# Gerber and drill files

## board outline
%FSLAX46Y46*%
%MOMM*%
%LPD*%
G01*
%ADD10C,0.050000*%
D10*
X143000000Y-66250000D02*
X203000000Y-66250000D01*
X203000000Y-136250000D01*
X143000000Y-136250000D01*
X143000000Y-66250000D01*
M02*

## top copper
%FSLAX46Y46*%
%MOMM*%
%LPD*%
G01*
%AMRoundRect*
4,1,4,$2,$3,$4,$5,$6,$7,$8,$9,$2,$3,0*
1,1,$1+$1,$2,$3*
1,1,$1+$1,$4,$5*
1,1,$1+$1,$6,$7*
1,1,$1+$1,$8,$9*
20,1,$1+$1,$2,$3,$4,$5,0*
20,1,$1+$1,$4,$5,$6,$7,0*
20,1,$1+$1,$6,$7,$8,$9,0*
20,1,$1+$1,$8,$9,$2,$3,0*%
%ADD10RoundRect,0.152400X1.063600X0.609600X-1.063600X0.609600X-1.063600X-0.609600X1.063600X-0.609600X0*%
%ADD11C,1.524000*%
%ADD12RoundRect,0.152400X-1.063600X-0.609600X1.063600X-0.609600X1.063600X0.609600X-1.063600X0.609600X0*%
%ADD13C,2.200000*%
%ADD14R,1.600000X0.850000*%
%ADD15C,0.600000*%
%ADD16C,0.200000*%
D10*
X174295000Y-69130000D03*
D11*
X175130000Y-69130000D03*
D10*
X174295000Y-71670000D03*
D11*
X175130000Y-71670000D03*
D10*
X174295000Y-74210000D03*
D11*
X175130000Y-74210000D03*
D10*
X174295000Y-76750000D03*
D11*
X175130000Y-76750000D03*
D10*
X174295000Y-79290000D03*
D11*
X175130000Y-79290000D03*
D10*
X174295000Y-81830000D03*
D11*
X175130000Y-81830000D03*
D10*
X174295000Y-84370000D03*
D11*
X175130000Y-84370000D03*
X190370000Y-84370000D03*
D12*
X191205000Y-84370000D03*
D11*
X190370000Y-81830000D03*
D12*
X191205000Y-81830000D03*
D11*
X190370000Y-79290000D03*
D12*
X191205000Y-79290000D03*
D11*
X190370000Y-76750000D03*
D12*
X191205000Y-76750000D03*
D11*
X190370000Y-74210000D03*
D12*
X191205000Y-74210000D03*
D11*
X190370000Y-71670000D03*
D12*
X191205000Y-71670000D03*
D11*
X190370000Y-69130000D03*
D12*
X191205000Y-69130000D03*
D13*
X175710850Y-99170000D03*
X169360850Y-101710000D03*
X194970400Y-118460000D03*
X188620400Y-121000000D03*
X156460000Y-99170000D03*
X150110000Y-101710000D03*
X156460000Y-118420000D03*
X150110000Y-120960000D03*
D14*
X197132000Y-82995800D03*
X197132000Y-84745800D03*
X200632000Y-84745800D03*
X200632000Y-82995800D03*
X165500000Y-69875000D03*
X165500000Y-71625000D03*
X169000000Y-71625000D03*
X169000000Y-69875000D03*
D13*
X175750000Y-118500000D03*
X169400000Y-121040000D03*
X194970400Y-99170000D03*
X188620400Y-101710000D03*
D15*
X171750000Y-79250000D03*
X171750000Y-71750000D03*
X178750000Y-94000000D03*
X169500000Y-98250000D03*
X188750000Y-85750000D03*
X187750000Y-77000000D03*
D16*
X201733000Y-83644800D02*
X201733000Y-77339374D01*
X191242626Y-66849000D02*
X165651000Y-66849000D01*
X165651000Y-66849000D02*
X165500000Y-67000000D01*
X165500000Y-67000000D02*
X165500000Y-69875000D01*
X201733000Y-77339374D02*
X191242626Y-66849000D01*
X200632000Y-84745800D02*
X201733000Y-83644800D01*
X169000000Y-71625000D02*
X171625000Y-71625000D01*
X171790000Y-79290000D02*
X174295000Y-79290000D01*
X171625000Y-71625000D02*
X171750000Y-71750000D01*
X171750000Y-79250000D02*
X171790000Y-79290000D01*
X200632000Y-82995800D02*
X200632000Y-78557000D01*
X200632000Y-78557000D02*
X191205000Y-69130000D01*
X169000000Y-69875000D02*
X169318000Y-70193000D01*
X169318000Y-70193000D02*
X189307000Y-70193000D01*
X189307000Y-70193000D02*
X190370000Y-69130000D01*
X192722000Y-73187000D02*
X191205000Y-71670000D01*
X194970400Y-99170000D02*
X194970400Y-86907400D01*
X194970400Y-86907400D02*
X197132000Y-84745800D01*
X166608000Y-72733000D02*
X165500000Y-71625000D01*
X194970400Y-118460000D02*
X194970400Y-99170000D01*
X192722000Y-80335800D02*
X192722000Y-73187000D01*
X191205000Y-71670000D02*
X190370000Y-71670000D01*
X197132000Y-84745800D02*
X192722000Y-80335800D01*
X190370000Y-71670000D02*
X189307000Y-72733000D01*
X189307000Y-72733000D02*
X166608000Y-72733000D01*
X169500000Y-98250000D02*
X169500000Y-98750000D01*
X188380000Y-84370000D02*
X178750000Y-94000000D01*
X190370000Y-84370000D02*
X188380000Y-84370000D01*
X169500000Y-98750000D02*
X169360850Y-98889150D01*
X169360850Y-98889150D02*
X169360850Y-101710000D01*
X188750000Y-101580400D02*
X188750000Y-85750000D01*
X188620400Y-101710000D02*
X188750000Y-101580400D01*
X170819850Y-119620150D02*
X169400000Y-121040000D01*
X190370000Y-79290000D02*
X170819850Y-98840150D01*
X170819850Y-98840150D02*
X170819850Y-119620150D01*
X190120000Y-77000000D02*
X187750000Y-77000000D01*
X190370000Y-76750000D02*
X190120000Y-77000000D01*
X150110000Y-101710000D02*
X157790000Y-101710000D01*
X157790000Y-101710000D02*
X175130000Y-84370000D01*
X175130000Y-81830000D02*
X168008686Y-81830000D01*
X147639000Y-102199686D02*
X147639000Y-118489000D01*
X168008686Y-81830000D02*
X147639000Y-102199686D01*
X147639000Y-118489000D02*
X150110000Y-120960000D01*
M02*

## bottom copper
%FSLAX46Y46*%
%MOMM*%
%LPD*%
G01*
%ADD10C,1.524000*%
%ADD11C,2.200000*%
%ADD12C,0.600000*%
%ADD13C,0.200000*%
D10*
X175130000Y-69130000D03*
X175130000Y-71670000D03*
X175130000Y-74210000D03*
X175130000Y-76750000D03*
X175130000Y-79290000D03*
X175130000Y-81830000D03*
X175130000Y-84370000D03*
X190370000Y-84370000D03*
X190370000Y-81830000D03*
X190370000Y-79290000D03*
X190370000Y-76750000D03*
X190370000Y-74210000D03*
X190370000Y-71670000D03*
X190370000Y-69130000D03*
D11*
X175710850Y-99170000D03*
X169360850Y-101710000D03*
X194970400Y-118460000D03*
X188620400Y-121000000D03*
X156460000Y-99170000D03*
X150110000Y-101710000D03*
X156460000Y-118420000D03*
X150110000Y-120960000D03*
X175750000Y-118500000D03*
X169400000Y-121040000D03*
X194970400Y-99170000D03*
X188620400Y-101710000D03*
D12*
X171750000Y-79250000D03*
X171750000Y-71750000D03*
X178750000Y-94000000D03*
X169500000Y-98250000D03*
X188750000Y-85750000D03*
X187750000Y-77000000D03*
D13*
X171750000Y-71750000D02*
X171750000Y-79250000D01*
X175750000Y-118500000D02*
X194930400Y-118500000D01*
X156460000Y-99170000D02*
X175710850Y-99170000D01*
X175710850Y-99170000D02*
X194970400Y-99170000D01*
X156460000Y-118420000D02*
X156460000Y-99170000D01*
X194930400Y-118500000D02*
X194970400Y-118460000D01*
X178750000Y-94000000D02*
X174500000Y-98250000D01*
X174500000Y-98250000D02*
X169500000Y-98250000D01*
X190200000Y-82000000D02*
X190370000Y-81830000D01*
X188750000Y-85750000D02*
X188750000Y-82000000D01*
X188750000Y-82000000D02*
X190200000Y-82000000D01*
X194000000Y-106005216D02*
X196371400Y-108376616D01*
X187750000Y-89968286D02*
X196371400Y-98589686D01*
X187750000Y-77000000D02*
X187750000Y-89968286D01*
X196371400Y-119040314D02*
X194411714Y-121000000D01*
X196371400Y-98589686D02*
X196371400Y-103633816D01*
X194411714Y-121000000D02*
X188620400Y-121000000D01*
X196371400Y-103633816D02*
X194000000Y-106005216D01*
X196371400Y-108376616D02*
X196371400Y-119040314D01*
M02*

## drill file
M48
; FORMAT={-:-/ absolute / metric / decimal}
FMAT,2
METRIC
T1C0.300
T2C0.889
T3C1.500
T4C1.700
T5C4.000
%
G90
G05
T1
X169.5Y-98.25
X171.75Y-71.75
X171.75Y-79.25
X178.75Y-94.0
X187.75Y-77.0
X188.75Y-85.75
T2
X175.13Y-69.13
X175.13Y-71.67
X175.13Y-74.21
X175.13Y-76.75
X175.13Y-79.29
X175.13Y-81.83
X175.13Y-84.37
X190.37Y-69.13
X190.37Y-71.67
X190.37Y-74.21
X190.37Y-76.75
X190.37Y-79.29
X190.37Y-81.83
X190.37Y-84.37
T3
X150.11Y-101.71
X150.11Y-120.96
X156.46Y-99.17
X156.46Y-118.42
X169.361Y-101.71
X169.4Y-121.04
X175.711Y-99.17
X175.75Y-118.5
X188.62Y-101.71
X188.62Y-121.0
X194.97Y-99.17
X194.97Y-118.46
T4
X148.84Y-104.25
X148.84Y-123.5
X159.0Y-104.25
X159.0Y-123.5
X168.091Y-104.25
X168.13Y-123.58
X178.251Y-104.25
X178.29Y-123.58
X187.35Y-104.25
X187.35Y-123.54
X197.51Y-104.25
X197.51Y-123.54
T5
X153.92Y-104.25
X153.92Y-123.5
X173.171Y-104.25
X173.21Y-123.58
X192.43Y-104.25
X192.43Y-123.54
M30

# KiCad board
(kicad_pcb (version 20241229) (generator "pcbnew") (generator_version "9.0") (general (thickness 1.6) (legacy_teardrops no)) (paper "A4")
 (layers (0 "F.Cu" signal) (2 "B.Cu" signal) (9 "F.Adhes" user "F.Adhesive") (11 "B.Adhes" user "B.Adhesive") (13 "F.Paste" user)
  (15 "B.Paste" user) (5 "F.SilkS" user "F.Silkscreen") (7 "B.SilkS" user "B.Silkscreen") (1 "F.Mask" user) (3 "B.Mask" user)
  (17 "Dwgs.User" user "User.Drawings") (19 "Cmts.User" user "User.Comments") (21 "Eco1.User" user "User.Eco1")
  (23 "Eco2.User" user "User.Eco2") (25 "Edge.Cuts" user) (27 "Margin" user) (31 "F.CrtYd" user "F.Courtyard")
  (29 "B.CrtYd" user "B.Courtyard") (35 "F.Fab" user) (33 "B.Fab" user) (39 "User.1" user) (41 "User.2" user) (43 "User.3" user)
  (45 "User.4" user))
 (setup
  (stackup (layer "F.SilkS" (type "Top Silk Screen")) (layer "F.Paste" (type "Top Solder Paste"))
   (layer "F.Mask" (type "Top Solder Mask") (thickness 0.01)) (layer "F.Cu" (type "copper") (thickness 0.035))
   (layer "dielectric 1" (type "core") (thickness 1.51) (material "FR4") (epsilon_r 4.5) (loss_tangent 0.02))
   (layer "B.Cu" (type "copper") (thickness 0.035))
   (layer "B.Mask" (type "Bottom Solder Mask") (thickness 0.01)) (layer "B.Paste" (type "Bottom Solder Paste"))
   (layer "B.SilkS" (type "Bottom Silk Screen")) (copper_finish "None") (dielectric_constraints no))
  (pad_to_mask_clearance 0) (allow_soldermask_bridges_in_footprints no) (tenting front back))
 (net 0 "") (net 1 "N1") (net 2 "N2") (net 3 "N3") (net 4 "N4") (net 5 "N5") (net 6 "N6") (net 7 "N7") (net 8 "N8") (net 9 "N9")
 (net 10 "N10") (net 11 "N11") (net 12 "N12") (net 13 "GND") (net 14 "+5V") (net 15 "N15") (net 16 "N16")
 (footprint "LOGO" (layer "F.Cu") (at 198.75 69.5)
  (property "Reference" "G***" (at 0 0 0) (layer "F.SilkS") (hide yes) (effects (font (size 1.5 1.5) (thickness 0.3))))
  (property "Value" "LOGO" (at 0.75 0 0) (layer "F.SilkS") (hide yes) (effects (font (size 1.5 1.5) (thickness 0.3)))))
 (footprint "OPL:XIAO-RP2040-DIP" (layer "F.Cu") (at 182.75 76.75)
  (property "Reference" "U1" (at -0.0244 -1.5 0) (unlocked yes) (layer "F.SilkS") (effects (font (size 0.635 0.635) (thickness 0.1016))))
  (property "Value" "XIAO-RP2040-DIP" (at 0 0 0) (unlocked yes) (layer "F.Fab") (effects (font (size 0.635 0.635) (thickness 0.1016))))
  (pad "1" smd roundrect (at -8.455 -7.62 180) (size 2.432 1.524) (layers "F.Cu" "F.Mask") (roundrect_rratio 0.1) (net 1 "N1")
   (thermal_bridge_angle 45))
  (pad "1" thru_hole circle (at -7.62 -7.62 180) (size 1.524 1.524) (drill 0.889) (layers "*.Cu" "*.Mask") (remove_unused_layers no)
   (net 1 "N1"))
  (pad "2" smd roundrect (at -8.455 -5.08 180) (size 2.432 1.524) (layers "F.Cu" "F.Mask") (roundrect_rratio 0.1) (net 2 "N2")
   (thermal_bridge_angle 45))
  (pad "2" thru_hole circle (at -7.62 -5.08 180) (size 1.524 1.524) (drill 0.889) (layers "*.Cu" "*.Mask") (remove_unused_layers no)
   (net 2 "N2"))
  (pad "3" smd roundrect (at -8.455 -2.54 180) (size 2.432 1.524) (layers "F.Cu" "F.Mask") (roundrect_rratio 0.1) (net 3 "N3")
   (thermal_bridge_angle 45))
  (pad "3" thru_hole circle (at -7.62 -2.54 180) (size 1.524 1.524) (drill 0.889) (layers "*.Cu" "*.Mask") (remove_unused_layers no)
   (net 3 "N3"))
  (pad "4" smd roundrect (at -8.455 0 180) (size 2.432 1.524) (layers "F.Cu" "F.Mask") (roundrect_rratio 0.1) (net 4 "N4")
   (thermal_bridge_angle 45))
  (pad "4" thru_hole circle (at -7.62 0 180) (size 1.524 1.524) (drill 0.889) (layers "*.Cu" "*.Mask") (remove_unused_layers no)
   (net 4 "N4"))
  (pad "5" smd roundrect (at -8.455 2.54 180) (size 2.432 1.524) (layers "F.Cu" "F.Mask") (roundrect_rratio 0.1) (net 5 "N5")
   (thermal_bridge_angle 45))
  (pad "5" thru_hole circle (at -7.62 2.54 180) (size 1.524 1.524) (drill 0.889) (layers "*.Cu" "*.Mask") (remove_unused_layers no)
   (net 5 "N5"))
  (pad "6" smd roundrect (at -8.455 5.08 180) (size 2.432 1.524) (layers "F.Cu" "F.Mask") (roundrect_rratio 0.1) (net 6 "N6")
   (thermal_bridge_angle 45))
  (pad "6" thru_hole circle (at -7.62 5.08 180) (size 1.524 1.524) (drill 0.889) (layers "*.Cu" "*.Mask") (remove_unused_layers no)
   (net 6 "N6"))
  (pad "7" smd roundrect (at -8.455 7.62 180) (size 2.432 1.524) (layers "F.Cu" "F.Mask") (roundrect_rratio 0.1) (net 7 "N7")
   (thermal_bridge_angle 45))
  (pad "7" thru_hole circle (at -7.62 7.62 180) (size 1.524 1.524) (drill 0.889) (layers "*.Cu" "*.Mask") (remove_unused_layers no)
   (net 7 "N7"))
  (pad "8" thru_hole circle (at 7.62 7.62) (size 1.524 1.524) (drill 0.889) (layers "*.Cu" "*.Mask") (remove_unused_layers no) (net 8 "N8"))
  (pad "8" smd roundrect (at 8.455 7.62) (size 2.432 1.524) (layers "F.Cu" "F.Mask") (roundrect_rratio 0.1) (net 8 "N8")
   (thermal_bridge_angle 45))
  (pad "9" thru_hole circle (at 7.62 5.08) (size 1.524 1.524) (drill 0.889) (layers "*.Cu" "*.Mask") (remove_unused_layers no) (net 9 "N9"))
  (pad "9" smd roundrect (at 8.455 5.08) (size 2.432 1.524) (layers "F.Cu" "F.Mask") (roundrect_rratio 0.1) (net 9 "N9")
   (thermal_bridge_angle 45))
  (pad "10" thru_hole circle (at 7.62 2.54) (size 1.524 1.524) (drill 0.889) (layers "*.Cu" "*.Mask") (remove_unused_layers no)
   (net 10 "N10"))
  (pad "10" smd roundrect (at 8.455 2.54) (size 2.432 1.524) (layers "F.Cu" "F.Mask") (roundrect_rratio 0.1) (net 10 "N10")
   (thermal_bridge_angle 45))
  (pad "11" thru_hole circle (at 7.62 0) (size 1.524 1.524) (drill 0.889) (layers "*.Cu" "*.Mask") (remove_unused_layers no) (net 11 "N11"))
  (pad "11" smd roundrect (at 8.455 0) (size 2.432 1.524) (layers "F.Cu" "F.Mask") (roundrect_rratio 0.1) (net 11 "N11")
   (thermal_bridge_angle 45))
  (pad "12" thru_hole circle (at 7.62 -2.54) (size 1.524 1.524) (drill 0.889) (layers "*.Cu" "*.Mask") (remove_unused_layers no)
   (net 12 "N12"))
  (pad "12" smd roundrect (at 8.455 -2.54) (size 2.432 1.524) (layers "F.Cu" "F.Mask") (roundrect_rratio 0.1) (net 12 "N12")
   (thermal_bridge_angle 45))
  (pad "13" thru_hole circle (at 7.62 -5.08) (size 1.524 1.524) (drill 0.889) (layers "*.Cu" "*.Mask") (remove_unused_layers no)
   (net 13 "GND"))
  (pad "13" smd roundrect (at 8.455 -5.08) (size 2.432 1.524) (layers "F.Cu" "F.Mask") (roundrect_rratio 0.1) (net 13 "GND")
   (thermal_bridge_angle 45))
  (pad "14" thru_hole circle (at 7.62 -7.62) (size 1.524 1.524) (drill 0.889) (layers "*.Cu" "*.Mask") (remove_unused_layers no)
   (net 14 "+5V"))
  (pad "14" smd roundrect (at 8.455 -7.62) (size 2.432 1.524) (layers "F.Cu" "F.Mask") (roundrect_rratio 0.1) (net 14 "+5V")
   (thermal_bridge_angle 45)))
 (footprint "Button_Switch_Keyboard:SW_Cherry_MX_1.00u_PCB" (layer "F.Cu") (at 175.71085 99.17)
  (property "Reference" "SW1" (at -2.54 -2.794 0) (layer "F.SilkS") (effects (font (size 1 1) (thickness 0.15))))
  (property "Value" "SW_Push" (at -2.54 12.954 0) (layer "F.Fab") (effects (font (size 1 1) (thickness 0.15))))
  (pad "" np_thru_hole circle (at -7.62 5.08) (size 1.7 1.7) (drill 1.7) (layers "*.Cu" "*.Mask"))
  (pad "" np_thru_hole circle (at -2.54 5.08) (size 4 4) (drill 4) (layers "*.Cu" "*.Mask"))
  (pad "" np_thru_hole circle (at 2.54 5.08) (size 1.7 1.7) (drill 1.7) (layers "*.Cu" "*.Mask"))
  (pad "1" thru_hole circle (at 0 0) (size 2.2 2.2) (drill 1.5) (layers "*.Cu" "*.Mask") (remove_unused_layers no) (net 13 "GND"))
  (pad "2" thru_hole circle (at -6.35 2.54) (size 2.2 2.2) (drill 1.5) (layers "*.Cu" "*.Mask") (remove_unused_layers no) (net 8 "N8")))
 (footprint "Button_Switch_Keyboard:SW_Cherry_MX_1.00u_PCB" (layer "F.Cu") (at 194.9704 118.46)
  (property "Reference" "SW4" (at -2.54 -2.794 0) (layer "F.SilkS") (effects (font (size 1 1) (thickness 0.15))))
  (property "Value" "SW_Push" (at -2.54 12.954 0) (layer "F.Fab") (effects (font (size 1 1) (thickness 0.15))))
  (pad "" np_thru_hole circle (at -7.62 5.08) (size 1.7 1.7) (drill 1.7) (layers "*.Cu" "*.Mask"))
  (pad "" np_thru_hole circle (at -2.54 5.08) (size 4 4) (drill 4) (layers "*.Cu" "*.Mask"))
  (pad "" np_thru_hole circle (at 2.54 5.08) (size 1.7 1.7) (drill 1.7) (layers "*.Cu" "*.Mask"))
  (pad "1" thru_hole circle (at 0 0) (size 2.2 2.2) (drill 1.5) (layers "*.Cu" "*.Mask") (remove_unused_layers no) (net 13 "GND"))
  (pad "2" thru_hole circle (at -6.35 2.54) (size 2.2 2.2) (drill 1.5) (layers "*.Cu" "*.Mask") (remove_unused_layers no) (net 11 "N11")))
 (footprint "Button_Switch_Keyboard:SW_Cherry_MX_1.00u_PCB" (layer "F.Cu") (at 156.46 99.17)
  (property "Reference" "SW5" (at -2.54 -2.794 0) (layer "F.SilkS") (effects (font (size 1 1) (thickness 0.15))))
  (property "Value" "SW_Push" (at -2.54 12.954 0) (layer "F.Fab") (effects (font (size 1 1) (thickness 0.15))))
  (pad "" np_thru_hole circle (at -7.62 5.08) (size 1.7 1.7) (drill 1.7) (layers "*.Cu" "*.Mask"))
  (pad "" np_thru_hole circle (at -2.54 5.08) (size 4 4) (drill 4) (layers "*.Cu" "*.Mask"))
  (pad "" np_thru_hole circle (at 2.54 5.08) (size 1.7 1.7) (drill 1.7) (layers "*.Cu" "*.Mask"))
  (pad "1" thru_hole circle (at 0 0) (size 2.2 2.2) (drill 1.5) (layers "*.Cu" "*.Mask") (remove_unused_layers no) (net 13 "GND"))
  (pad "2" thru_hole circle (at -6.35 2.54) (size 2.2 2.2) (drill 1.5) (layers "*.Cu" "*.Mask") (remove_unused_layers no) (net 7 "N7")))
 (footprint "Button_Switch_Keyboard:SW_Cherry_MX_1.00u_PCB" (layer "F.Cu") (at 156.46 118.42)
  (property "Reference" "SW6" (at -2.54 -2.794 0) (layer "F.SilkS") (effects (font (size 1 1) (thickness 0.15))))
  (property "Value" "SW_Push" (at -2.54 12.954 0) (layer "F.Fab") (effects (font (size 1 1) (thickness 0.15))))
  (pad "" np_thru_hole circle (at -7.62 5.08) (size 1.7 1.7) (drill 1.7) (layers "*.Cu" "*.Mask"))
  (pad "" np_thru_hole circle (at -2.54 5.08) (size 4 4) (drill 4) (layers "*.Cu" "*.Mask"))
  (pad "" np_thru_hole circle (at 2.54 5.08) (size 1.7 1.7) (drill 1.7) (layers "*.Cu" "*.Mask"))
  (pad "1" thru_hole circle (at 0 0) (size 2.2 2.2) (drill 1.5) (layers "*.Cu" "*.Mask") (remove_unused_layers no) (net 13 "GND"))
  (pad "2" thru_hole circle (at -6.35 2.54) (size 2.2 2.2) (drill 1.5) (layers "*.Cu" "*.Mask") (remove_unused_layers no) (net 6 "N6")))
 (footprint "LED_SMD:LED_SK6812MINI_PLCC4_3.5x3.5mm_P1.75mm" (layer "F.Cu") (at 198.882 83.8708)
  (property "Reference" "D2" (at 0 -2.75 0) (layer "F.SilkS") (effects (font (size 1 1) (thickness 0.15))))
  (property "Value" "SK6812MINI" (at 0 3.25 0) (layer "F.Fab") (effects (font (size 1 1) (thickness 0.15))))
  (pad "1" smd rect (at -1.75 -0.875) (size 1.6 0.85) (layers "F.Cu" "F.Mask" "F.Paste") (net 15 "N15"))
  (pad "2" smd rect (at -1.75 0.875) (size 1.6 0.85) (layers "F.Cu" "F.Mask" "F.Paste") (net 13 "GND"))
  (pad "3" smd rect (at 1.75 0.875) (size 1.6 0.85) (layers "F.Cu" "F.Mask" "F.Paste") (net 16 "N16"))
  (pad "4" smd rect (at 1.75 -0.875) (size 1.6 0.85) (layers "F.Cu" "F.Mask" "F.Paste") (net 14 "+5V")))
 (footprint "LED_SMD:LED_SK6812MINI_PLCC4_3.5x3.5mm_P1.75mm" (layer "F.Cu") (at 167.25 70.75)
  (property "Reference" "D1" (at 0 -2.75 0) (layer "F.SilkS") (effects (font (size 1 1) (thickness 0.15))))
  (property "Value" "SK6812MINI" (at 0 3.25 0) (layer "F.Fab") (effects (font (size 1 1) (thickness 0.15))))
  (pad "1" smd rect (at -1.75 -0.875) (size 1.6 0.85) (layers "F.Cu" "F.Mask" "F.Paste") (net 16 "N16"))
  (pad "2" smd rect (at -1.75 0.875) (size 1.6 0.85) (layers "F.Cu" "F.Mask" "F.Paste") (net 13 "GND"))
  (pad "3" smd rect (at 1.75 0.875) (size 1.6 0.85) (layers "F.Cu" "F.Mask" "F.Paste") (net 5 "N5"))
  (pad "4" smd rect (at 1.75 -0.875) (size 1.6 0.85) (layers "F.Cu" "F.Mask" "F.Paste") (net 14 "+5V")))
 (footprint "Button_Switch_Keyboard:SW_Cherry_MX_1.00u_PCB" (layer "F.Cu") (at 175.75 118.5)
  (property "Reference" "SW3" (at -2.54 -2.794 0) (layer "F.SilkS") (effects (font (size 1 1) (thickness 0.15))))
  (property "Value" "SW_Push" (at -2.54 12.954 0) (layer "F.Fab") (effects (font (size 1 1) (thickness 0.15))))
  (pad "" np_thru_hole circle (at -7.62 5.08) (size 1.7 1.7) (drill 1.7) (layers "*.Cu" "*.Mask"))
  (pad "" np_thru_hole circle (at -2.54 5.08) (size 4 4) (drill 4) (layers "*.Cu" "*.Mask"))
  (pad "" np_thru_hole circle (at 2.54 5.08) (size 1.7 1.7) (drill 1.7) (layers "*.Cu" "*.Mask"))
  (pad "1" thru_hole circle (at 0 0) (size 2.2 2.2) (drill 1.5) (layers "*.Cu" "*.Mask") (remove_unused_layers no) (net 13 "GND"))
  (pad "2" thru_hole circle (at -6.35 2.54) (size 2.2 2.2) (drill 1.5) (layers "*.Cu" "*.Mask") (remove_unused_layers no) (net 10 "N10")))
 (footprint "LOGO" (layer "F.Cu") (at 147.25 72)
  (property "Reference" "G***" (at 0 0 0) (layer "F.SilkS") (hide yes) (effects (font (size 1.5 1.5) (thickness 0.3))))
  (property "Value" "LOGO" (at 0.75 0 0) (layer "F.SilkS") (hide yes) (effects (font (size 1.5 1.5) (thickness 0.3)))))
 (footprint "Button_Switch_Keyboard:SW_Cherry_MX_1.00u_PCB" (layer "F.Cu") (at 194.9704 99.17)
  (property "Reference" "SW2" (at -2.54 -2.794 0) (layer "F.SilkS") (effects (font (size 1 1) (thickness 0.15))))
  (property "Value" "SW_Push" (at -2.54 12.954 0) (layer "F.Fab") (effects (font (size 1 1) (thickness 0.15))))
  (pad "" np_thru_hole circle (at -7.62 5.08) (size 1.7 1.7) (drill 1.7) (layers "*.Cu" "*.Mask"))
  (pad "" np_thru_hole circle (at -2.54 5.08) (size 4 4) (drill 4) (layers "*.Cu" "*.Mask"))
  (pad "" np_thru_hole circle (at 2.54 5.08) (size 1.7 1.7) (drill 1.7) (layers "*.Cu" "*.Mask"))
  (pad "1" thru_hole circle (at 0 0) (size 2.2 2.2) (drill 1.5) (layers "*.Cu" "*.Mask") (remove_unused_layers no) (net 13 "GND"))
  (pad "2" thru_hole circle (at -6.35 2.54) (size 2.2 2.2) (drill 1.5) (layers "*.Cu" "*.Mask") (remove_unused_layers no) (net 9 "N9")))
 (gr_rect (start 143 66.25) (end 203 136.25) (stroke (width 0.05) (type solid)) (fill no) (layer "Edge.Cuts"))
 (segment (start 201.733 83.6448) (end 201.733 77.339374) (width 0.2) (layer "F.Cu") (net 16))
 (segment (start 191.242626 66.849) (end 165.651 66.849) (width 0.2) (layer "F.Cu") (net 16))
 (segment (start 165.651 66.849) (end 165.5 67) (width 0.2) (layer "F.Cu") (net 16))
 (segment (start 165.5 67) (end 165.5 69.875) (width 0.2) (layer "F.Cu") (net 16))
 (segment (start 201.733 77.339374) (end 191.242626 66.849) (width 0.2) (layer "F.Cu") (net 16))
 (segment (start 200.632 84.7458) (end 201.733 83.6448) (width 0.2) (layer "F.Cu") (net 16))
 (segment (start 169 71.625) (end 171.625 71.625) (width 0.2) (layer "F.Cu") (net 5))
 (segment (start 171.79 79.29) (end 174.295 79.29) (width 0.2) (layer "F.Cu") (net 5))
 (segment (start 171.625 71.625) (end 171.75 71.75) (width 0.2) (layer "F.Cu") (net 5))
 (segment (start 171.75 79.25) (end 171.79 79.29) (width 0.2) (layer "F.Cu") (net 5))
 (via (at 171.75 79.25) (size 0.6) (drill 0.3) (layers "F.Cu" "B.Cu") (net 5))
 (via (at 171.75 71.75) (size 0.6) (drill 0.3) (layers "F.Cu" "B.Cu") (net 5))
 (segment (start 171.75 71.75) (end 171.75 79.25) (width 0.2) (layer "B.Cu") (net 5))
 (segment (start 200.632 82.9958) (end 200.632 78.557) (width 0.2) (layer "F.Cu") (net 14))
 (segment (start 200.632 78.557) (end 191.205 69.13) (width 0.2) (layer "F.Cu") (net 14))
 (segment (start 169 69.875) (end 169.318 70.193) (width 0.2) (layer "F.Cu") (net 14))
 (segment (start 169.318 70.193) (end 189.307 70.193) (width 0.2) (layer "F.Cu") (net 14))
 (segment (start 189.307 70.193) (end 190.37 69.13) (width 0.2) (layer "F.Cu") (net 14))
 (segment (start 192.722 73.187) (end 191.205 71.67) (width 0.2) (layer "F.Cu") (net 13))
 (segment (start 194.9704 99.17) (end 194.9704 86.9074) (width 0.2) (layer "F.Cu") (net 13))
 (segment (start 194.9704 86.9074) (end 197.132 84.7458) (width 0.2) (layer "F.Cu") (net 13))
 (segment (start 166.608 72.733) (end 165.5 71.625) (width 0.2) (layer "F.Cu") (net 13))
 (segment (start 194.9704 118.46) (end 194.9704 99.17) (width 0.2) (layer "F.Cu") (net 13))
 (segment (start 192.722 80.3358) (end 192.722 73.187) (width 0.2) (layer "F.Cu") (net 13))
 (segment (start 191.205 71.67) (end 190.37 71.67) (width 0.2) (layer "F.Cu") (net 13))
 (segment (start 197.132 84.7458) (end 192.722 80.3358) (width 0.2) (layer "F.Cu") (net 13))
 (segment (start 190.37 71.67) (end 189.307 72.733) (width 0.2) (layer "F.Cu") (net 13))
 (segment (start 189.307 72.733) (end 166.608 72.733) (width 0.2) (layer "F.Cu") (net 13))
 (segment (start 175.75 118.5) (end 194.9304 118.5) (width 0.2) (layer "B.Cu") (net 13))
 (segment (start 156.46 99.17) (end 175.71085 99.17) (width 0.2) (layer "B.Cu") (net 13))
 (segment (start 175.71085 99.17) (end 194.9704 99.17) (width 0.2) (layer "B.Cu") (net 13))
 (segment (start 156.46 118.42) (end 156.46 99.17) (width 0.2) (layer "B.Cu") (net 13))
 (segment (start 194.9304 118.5) (end 194.9704 118.46) (width 0.2) (layer "B.Cu") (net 13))
 (segment (start 169.5 98.25) (end 169.5 98.75) (width 0.2) (layer "F.Cu") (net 8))
 (segment (start 188.38 84.37) (end 178.75 94) (width 0.2) (layer "F.Cu") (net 8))
 (segment (start 190.37 84.37) (end 188.38 84.37) (width 0.2) (layer "F.Cu") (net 8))
 (segment (start 169.5 98.75) (end 169.36085 98.88915) (width 0.2) (layer "F.Cu") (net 8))
 (segment (start 169.36085 98.88915) (end 169.36085 101.71) (width 0.2) (layer "F.Cu") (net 8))
 (via (at 178.75 94) (size 0.6) (drill 0.3) (layers "F.Cu" "B.Cu") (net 8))
 (via (at 169.5 98.25) (size 0.6) (drill 0.3) (layers "F.Cu" "B.Cu") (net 8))
 (segment (start 178.75 94) (end 174.5 98.25) (width 0.2) (layer "B.Cu") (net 8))
 (segment (start 174.5 98.25) (end 169.5 98.25) (width 0.2) (layer "B.Cu") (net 8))
 (segment (start 188.75 101.5804) (end 188.75 85.75) (width 0.2) (layer "F.Cu") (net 9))
 (segment (start 188.6204 101.71) (end 188.75 101.5804) (width 0.2) (layer "F.Cu") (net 9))
 (via (at 188.75 85.75) (size 0.6) (drill 0.3) (layers "F.Cu" "B.Cu") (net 9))
 (segment (start 190.2 82) (end 190.37 81.83) (width 0.2) (layer "B.Cu") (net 9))
 (segment (start 188.75 85.75) (end 188.75 82) (width 0.2) (layer "B.Cu") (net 9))
 (segment (start 188.75 82) (end 190.2 82) (width 0.2) (layer "B.Cu") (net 9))
 (segment (start 170.81985 119.62015) (end 169.4 121.04) (width 0.2) (layer "F.Cu") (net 10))
 (segment (start 190.37 79.29) (end 170.81985 98.84015) (width 0.2) (layer "F.Cu") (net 10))
 (segment (start 170.81985 98.84015) (end 170.81985 119.62015) (width 0.2) (layer "F.Cu") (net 10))
 (segment (start 190.12 77) (end 187.75 77) (width 0.2) (layer "F.Cu") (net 11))
 (segment (start 190.37 76.75) (end 190.12 77) (width 0.2) (layer "F.Cu") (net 11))
 (via (at 187.75 77) (size 0.6) (drill 0.3) (layers "F.Cu" "B.Cu") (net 11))
 (segment (start 194 106.005216) (end 196.3714 108.376616) (width 0.2) (layer "B.Cu") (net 11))
 (segment (start 187.75 89.968286) (end 196.3714 98.589686) (width 0.2) (layer "B.Cu") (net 11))
 (segment (start 187.75 77) (end 187.75 89.968286) (width 0.2) (layer "B.Cu") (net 11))
 (segment (start 196.3714 119.040314) (end 194.411714 121) (width 0.2) (layer "B.Cu") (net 11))
 (segment (start 196.3714 98.589686) (end 196.3714 103.633816) (width 0.2) (layer "B.Cu") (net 11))
 (segment (start 194.411714 121) (end 188.6204 121) (width 0.2) (layer "B.Cu") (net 11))
 (segment (start 196.3714 103.633816) (end 194 106.005216) (width 0.2) (layer "B.Cu") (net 11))
 (segment (start 196.3714 108.376616) (end 196.3714 119.040314) (width 0.2) (layer "B.Cu") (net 11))
 (segment (start 150.11 101.71) (end 157.79 101.71) (width 0.2) (layer "F.Cu") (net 7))
 (segment (start 157.79 101.71) (end 175.13 84.37) (width 0.2) (layer "F.Cu") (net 7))
 (segment (start 175.13 81.83) (end 168.008686 81.83) (width 0.2) (layer "F.Cu") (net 6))
 (segment (start 147.639 102.199686) (end 147.639 118.489) (width 0.2) (layer "F.Cu") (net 6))
 (segment (start 168.008686 81.83) (end 147.639 102.199686) (width 0.2) (layer "F.Cu") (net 6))
 (segment (start 147.639 118.489) (end 150.11 120.96) (width 0.2) (layer "F.Cu") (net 6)))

